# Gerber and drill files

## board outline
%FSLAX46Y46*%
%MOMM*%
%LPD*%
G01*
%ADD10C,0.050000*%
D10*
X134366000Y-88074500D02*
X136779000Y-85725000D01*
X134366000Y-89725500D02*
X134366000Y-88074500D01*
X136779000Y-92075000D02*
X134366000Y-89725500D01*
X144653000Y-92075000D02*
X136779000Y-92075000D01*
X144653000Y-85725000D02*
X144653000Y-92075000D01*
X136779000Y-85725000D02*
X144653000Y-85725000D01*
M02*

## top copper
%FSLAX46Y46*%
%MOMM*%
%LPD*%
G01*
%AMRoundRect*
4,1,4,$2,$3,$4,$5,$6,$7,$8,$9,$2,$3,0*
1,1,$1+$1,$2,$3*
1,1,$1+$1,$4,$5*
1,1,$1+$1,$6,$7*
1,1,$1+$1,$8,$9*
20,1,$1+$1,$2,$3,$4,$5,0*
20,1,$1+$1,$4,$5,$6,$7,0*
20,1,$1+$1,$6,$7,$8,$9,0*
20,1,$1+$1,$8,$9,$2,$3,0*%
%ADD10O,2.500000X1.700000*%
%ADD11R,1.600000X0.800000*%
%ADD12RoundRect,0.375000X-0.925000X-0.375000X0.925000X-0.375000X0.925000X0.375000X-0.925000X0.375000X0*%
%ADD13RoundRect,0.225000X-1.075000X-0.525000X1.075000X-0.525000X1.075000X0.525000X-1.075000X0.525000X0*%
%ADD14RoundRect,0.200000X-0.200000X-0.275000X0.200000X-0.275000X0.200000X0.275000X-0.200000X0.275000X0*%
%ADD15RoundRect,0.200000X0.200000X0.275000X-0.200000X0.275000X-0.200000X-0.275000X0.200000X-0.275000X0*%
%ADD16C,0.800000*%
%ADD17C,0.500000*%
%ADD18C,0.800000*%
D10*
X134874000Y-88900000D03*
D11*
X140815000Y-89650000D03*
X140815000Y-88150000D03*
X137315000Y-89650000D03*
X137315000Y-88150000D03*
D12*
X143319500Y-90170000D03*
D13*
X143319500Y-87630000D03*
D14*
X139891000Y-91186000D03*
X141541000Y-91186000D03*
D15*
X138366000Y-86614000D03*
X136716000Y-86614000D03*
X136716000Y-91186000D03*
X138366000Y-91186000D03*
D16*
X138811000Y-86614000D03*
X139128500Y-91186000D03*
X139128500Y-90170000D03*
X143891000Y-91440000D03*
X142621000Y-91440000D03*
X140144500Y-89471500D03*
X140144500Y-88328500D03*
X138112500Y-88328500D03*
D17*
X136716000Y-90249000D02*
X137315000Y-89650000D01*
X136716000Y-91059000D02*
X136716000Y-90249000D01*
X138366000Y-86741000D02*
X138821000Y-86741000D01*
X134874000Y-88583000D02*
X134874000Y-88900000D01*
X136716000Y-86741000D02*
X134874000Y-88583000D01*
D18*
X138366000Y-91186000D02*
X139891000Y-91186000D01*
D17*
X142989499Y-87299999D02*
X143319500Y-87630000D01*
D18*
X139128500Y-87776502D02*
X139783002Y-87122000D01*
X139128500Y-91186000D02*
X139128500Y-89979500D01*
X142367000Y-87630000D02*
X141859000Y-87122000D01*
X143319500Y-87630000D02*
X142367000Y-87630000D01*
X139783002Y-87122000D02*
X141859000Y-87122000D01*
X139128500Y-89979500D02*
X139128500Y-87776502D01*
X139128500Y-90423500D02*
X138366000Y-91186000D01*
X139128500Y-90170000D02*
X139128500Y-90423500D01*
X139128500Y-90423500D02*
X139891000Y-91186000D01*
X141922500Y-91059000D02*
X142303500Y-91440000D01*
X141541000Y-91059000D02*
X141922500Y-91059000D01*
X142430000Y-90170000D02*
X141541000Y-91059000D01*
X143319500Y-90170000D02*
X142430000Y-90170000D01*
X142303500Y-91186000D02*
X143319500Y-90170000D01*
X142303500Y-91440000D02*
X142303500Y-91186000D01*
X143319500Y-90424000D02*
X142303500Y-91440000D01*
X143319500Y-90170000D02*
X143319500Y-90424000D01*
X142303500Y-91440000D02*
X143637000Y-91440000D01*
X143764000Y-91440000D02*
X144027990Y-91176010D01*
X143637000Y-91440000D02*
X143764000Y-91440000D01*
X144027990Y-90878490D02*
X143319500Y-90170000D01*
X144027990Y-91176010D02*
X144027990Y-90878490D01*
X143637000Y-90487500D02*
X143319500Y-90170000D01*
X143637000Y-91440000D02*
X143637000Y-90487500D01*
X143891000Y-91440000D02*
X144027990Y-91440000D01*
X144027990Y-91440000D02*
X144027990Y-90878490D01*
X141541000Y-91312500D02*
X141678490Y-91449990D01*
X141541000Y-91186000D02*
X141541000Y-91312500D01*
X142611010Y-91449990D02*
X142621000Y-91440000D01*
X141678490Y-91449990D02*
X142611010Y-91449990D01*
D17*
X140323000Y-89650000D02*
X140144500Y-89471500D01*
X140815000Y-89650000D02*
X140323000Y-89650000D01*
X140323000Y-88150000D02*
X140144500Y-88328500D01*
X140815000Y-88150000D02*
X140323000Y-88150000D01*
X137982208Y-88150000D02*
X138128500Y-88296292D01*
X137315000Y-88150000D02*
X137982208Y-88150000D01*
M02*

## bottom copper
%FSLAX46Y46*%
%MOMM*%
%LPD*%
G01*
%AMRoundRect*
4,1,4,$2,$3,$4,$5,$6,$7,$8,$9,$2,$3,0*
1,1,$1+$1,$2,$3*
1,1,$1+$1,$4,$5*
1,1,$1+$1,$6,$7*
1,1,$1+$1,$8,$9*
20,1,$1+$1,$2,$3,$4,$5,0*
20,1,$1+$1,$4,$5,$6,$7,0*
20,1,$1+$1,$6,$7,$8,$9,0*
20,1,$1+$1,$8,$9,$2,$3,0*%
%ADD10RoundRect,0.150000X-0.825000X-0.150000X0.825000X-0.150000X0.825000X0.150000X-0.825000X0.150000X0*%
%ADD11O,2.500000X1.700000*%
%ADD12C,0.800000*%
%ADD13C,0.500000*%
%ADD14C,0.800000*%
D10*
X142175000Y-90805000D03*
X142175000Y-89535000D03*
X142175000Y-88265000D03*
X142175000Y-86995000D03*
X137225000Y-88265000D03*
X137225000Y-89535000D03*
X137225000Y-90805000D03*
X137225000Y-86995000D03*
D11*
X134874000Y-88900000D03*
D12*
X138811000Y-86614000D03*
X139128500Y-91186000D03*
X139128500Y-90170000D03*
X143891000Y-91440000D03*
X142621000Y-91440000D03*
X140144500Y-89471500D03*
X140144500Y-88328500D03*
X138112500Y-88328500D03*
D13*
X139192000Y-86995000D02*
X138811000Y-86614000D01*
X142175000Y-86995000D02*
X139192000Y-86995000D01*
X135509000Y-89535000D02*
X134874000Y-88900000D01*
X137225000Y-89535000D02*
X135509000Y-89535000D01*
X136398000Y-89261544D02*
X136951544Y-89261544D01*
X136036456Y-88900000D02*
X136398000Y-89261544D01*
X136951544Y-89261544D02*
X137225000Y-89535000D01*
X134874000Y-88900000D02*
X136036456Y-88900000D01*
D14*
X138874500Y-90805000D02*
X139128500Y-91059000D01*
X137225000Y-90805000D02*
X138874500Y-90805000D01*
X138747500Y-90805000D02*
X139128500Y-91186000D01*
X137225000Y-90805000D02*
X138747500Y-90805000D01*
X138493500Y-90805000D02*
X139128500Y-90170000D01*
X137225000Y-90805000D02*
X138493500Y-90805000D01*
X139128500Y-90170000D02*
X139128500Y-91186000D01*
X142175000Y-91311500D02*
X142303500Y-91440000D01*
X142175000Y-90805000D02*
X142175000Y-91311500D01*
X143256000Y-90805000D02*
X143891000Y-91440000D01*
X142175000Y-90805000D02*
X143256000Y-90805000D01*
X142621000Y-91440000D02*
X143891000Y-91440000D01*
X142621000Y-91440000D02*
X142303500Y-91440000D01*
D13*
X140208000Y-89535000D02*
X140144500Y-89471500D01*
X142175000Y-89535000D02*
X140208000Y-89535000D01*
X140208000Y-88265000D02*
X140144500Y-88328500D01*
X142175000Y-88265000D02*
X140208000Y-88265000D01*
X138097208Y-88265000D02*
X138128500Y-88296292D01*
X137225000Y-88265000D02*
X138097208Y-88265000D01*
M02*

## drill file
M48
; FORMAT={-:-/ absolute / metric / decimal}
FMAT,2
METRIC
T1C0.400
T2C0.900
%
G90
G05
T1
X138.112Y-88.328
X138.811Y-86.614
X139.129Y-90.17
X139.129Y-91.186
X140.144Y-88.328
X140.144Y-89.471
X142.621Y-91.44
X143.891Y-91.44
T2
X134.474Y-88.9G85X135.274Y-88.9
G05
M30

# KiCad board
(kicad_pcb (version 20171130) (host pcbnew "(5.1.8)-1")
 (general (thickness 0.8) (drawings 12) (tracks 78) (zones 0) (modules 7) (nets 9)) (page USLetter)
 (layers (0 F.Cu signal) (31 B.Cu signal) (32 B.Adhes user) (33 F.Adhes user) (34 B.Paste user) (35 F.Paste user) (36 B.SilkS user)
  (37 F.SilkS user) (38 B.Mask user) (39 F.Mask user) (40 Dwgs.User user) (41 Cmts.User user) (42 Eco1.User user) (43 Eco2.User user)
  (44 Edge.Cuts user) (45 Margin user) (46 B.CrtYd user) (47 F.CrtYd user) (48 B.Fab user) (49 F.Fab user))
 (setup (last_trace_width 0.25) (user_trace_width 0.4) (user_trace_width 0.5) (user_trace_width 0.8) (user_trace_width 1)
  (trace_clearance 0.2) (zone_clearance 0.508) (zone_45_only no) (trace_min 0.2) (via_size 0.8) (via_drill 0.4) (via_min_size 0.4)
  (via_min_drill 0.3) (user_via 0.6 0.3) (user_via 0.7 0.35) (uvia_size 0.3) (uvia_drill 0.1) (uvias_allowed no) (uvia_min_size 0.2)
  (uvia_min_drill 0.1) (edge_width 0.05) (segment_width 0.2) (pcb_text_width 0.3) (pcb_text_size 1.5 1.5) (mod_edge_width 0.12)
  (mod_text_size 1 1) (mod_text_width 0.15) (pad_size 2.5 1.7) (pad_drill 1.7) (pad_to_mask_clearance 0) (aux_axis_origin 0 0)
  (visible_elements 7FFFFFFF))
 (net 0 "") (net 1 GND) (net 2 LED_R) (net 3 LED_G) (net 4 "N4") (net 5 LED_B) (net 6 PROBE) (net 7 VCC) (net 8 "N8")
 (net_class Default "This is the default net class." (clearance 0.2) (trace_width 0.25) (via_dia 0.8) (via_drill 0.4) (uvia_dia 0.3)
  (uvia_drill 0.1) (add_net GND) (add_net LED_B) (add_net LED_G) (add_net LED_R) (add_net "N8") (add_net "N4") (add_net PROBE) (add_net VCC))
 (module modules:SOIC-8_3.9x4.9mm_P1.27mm (layer B.Cu) (at 139.7 88.9)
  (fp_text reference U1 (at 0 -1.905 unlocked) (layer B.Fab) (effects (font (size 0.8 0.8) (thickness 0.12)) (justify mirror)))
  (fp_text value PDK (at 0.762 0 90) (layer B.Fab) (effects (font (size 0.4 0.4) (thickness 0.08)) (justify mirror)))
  (pad 8 smd roundrect (at 2.475 1.905) (size 1.95 0.6) (layers B.Cu B.Paste B.Mask) (roundrect_rratio 0.25) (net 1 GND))
  (pad 7 smd roundrect (at 2.475 0.635) (size 1.95 0.6) (layers B.Cu B.Paste B.Mask) (roundrect_rratio 0.25) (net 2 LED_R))
  (pad 6 smd roundrect (at 2.475 -0.635) (size 1.95 0.6) (layers B.Cu B.Paste B.Mask) (roundrect_rratio 0.25) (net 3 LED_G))
  (pad 5 smd roundrect (at 2.475 -1.905) (size 1.95 0.6) (layers B.Cu B.Paste B.Mask) (roundrect_rratio 0.25) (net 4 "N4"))
  (pad 3 smd roundrect (at -2.475 -0.635) (size 1.95 0.6) (layers B.Cu B.Paste B.Mask) (roundrect_rratio 0.25) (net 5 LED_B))
  (pad 2 smd roundrect (at -2.475 0.635) (size 1.95 0.6) (layers B.Cu B.Paste B.Mask) (roundrect_rratio 0.25) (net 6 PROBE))
  (pad 1 smd roundrect (at -2.475 1.905) (size 1.95 0.6) (layers B.Cu B.Paste B.Mask) (roundrect_rratio 0.25) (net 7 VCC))
  (pad 4 smd roundrect (at -2.475 -1.905) (size 1.95 0.6) (layers B.Cu B.Paste B.Mask) (roundrect_rratio 0.25)))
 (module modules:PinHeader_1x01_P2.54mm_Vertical (layer B.Cu) (at 134.874 88.9)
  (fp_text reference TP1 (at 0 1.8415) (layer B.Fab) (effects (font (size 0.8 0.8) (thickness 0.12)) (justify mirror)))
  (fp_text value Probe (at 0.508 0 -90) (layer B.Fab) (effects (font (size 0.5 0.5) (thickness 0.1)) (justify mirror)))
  (pad 1 thru_hole oval (at 0 0) (size 2.5 1.7) (drill oval 1.7 0.9) (layers *.Cu *.Mask) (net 6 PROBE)))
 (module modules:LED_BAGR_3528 (layer F.Cu) (at 139.065 88.9 180)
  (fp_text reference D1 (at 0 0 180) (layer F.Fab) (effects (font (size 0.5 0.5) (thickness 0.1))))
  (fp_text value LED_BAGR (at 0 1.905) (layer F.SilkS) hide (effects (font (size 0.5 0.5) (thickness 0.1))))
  (pad 4 smd rect (at -1.75 -0.75 180) (size 1.6 0.8) (layers F.Cu F.Paste F.Mask) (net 2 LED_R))
  (pad 3 smd rect (at -1.75 0.75 180) (size 1.6 0.8) (layers F.Cu F.Paste F.Mask) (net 3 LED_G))
  (pad 2 smd rect (at 1.75 -0.75 180) (size 1.6 0.8) (layers F.Cu F.Paste F.Mask) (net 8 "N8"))
  (pad 1 smd rect (at 1.75 0.75 180) (size 1.6 0.8) (layers F.Cu F.Paste F.Mask) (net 5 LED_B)))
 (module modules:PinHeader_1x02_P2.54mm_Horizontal (layer F.Cu) (at 143.3195 87.63)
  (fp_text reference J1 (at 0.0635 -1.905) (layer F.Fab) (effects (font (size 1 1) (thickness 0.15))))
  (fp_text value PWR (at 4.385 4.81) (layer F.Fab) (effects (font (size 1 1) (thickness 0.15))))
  (pad 1 smd roundrect (at 0 2.54) (size 2.6 1.5) (layers F.Cu F.Paste F.Mask) (roundrect_rratio 0.25) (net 1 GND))
  (pad 2 smd roundrect (at 0 0) (size 2.6 1.5) (layers F.Cu F.Paste F.Mask) (roundrect_rratio 0.15) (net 7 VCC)))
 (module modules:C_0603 (layer F.Cu) (at 140.716 91.186)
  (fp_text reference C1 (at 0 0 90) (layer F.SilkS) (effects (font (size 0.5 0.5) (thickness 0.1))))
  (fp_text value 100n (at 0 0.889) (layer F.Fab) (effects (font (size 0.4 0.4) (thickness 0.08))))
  (pad 1 smd roundrect (at -0.825 0) (size 0.8 0.95) (layers F.Cu F.Paste F.Mask) (roundrect_rratio 0.25) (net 7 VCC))
  (pad 2 smd roundrect (at 0.825 0) (size 0.8 0.95) (layers F.Cu F.Paste F.Mask) (roundrect_rratio 0.25) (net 1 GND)))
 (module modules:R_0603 (layer F.Cu) (at 137.541 86.614 180)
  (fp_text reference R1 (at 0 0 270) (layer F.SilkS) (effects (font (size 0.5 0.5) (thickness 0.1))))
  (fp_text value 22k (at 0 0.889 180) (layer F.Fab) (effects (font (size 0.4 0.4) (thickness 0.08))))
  (pad 1 smd roundrect (at -0.825 0 180) (size 0.8 0.95) (layers F.Cu F.Paste F.Mask) (roundrect_rratio 0.25) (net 4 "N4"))
  (pad 2 smd roundrect (at 0.825 0 180) (size 0.8 0.95) (layers F.Cu F.Paste F.Mask) (roundrect_rratio 0.25) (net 6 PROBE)))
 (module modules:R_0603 (layer F.Cu) (at 137.541 91.186 180)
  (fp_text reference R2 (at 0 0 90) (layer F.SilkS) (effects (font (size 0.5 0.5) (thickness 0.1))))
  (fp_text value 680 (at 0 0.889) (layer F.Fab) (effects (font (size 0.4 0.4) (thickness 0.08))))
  (pad 2 smd roundrect (at 0.825 0 180) (size 0.8 0.95) (layers F.Cu F.Paste F.Mask) (roundrect_rratio 0.25) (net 8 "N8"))
  (pad 1 smd roundrect (at -0.825 0 180) (size 0.8 0.95) (layers F.Cu F.Paste F.Mask) (roundrect_rratio 0.25) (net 7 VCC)))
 (gr_line (start 134.366 88.0745) (end 136.779 85.725) (layer Edge.Cuts) (width 0.05))
 (gr_line (start 134.366 89.7255) (end 134.366 88.0745) (layer Edge.Cuts) (width 0.05))
 (gr_line (start 136.779 92.075) (end 134.366 89.7255) (layer Edge.Cuts) (width 0.05))
 (gr_line (start 144.653 92.075) (end 136.779 92.075) (layer Edge.Cuts) (width 0.05))
 (gr_line (start 144.653 85.725) (end 144.653 92.075) (layer Edge.Cuts) (width 0.05))
 (gr_line (start 136.779 85.725) (end 144.653 85.725) (layer Edge.Cuts) (width 0.05))
 (segment (start 136.716 90.249) (end 137.315 89.65) (width 0.5) (layer F.Cu) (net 8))
 (segment (start 136.716 91.059) (end 136.716 90.249) (width 0.5) (layer F.Cu) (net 8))
 (via (at 138.811 86.614) (size 0.8) (drill 0.4) (layers F.Cu B.Cu) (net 4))
 (segment (start 138.366 86.741) (end 138.821 86.741) (width 0.5) (layer F.Cu) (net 4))
 (segment (start 139.192 86.995) (end 138.811 86.614) (width 0.5) (layer B.Cu) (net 4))
 (segment (start 142.175 86.995) (end 139.192 86.995) (width 0.5) (layer B.Cu) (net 4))
 (segment (start 135.509 89.535) (end 134.874 88.9) (width 0.5) (layer B.Cu) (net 6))
 (segment (start 137.225 89.535) (end 135.509 89.535) (width 0.5) (layer B.Cu) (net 6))
 (segment (start 136.398 89.261544) (end 136.951544 89.261544) (width 0.5) (layer B.Cu) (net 6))
 (segment (start 136.036456 88.9) (end 136.398 89.261544) (width 0.5) (layer B.Cu) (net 6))
 (segment (start 136.951544 89.261544) (end 137.225 89.535) (width 0.5) (layer B.Cu) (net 6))
 (segment (start 134.874 88.9) (end 136.036456 88.9) (width 0.5) (layer B.Cu) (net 6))
 (segment (start 134.874 88.583) (end 134.874 88.9) (width 0.5) (layer F.Cu) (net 6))
 (segment (start 136.716 86.741) (end 134.874 88.583) (width 0.5) (layer F.Cu) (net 6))
 (via (at 139.1285 91.186) (size 0.8) (drill 0.4) (layers F.Cu B.Cu) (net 7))
 (segment (start 138.8745 90.805) (end 139.1285 91.059) (width 0.8) (layer B.Cu) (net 7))
 (segment (start 137.225 90.805) (end 138.8745 90.805) (width 0.8) (layer B.Cu) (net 7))
 (segment (start 138.366 91.186) (end 139.891 91.186) (width 0.8) (layer F.Cu) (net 7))
 (segment (start 142.989499 87.299999) (end 143.3195 87.63) (width 0.5) (layer F.Cu) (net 7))
 (segment (start 139.1285 87.776502) (end 139.783002 87.122) (width 0.8) (layer F.Cu) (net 7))
 (segment (start 139.1285 91.186) (end 139.1285 89.9795) (width 0.8) (layer F.Cu) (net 7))
 (segment (start 142.367 87.63) (end 141.859 87.122) (width 0.8) (layer F.Cu) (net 7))
 (segment (start 143.3195 87.63) (end 142.367 87.63) (width 0.8) (layer F.Cu) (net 7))
 (segment (start 139.783002 87.122) (end 141.859 87.122) (width 0.8) (layer F.Cu) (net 7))
 (segment (start 139.1285 89.9795) (end 139.1285 87.776502) (width 0.8) (layer F.Cu) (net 7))
 (via (at 139.1285 90.17) (size 0.8) (drill 0.4) (layers F.Cu B.Cu) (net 7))
 (segment (start 138.7475 90.805) (end 139.1285 91.186) (width 0.8) (layer B.Cu) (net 7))
 (segment (start 137.225 90.805) (end 138.7475 90.805) (width 0.8) (layer B.Cu) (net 7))
 (segment (start 138.4935 90.805) (end 139.1285 90.17) (width 0.8) (layer B.Cu) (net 7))
 (segment (start 137.225 90.805) (end 138.4935 90.805) (width 0.8) (layer B.Cu) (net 7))
 (segment (start 139.1285 90.17) (end 139.1285 91.186) (width 0.8) (layer B.Cu) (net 7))
 (segment (start 139.1285 90.4235) (end 138.366 91.186) (width 0.8) (layer F.Cu) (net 7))
 (segment (start 139.1285 90.17) (end 139.1285 90.4235) (width 0.8) (layer F.Cu) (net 7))
 (segment (start 139.1285 90.4235) (end 139.891 91.186) (width 0.8) (layer F.Cu) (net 7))
 (via (at 143.891 91.44) (size 0.8) (drill 0.4) (layers F.Cu B.Cu) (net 1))
 (via (at 142.621 91.44) (size 0.8) (drill 0.4) (layers F.Cu B.Cu) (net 1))
 (segment (start 142.175 91.3115) (end 142.3035 91.44) (width 0.8) (layer B.Cu) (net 1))
 (segment (start 142.175 90.805) (end 142.175 91.3115) (width 0.8) (layer B.Cu) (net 1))
 (segment (start 141.9225 91.059) (end 142.3035 91.44) (width 0.8) (layer F.Cu) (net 1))
 (segment (start 141.541 91.059) (end 141.9225 91.059) (width 0.8) (layer F.Cu) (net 1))
 (segment (start 142.43 90.17) (end 141.541 91.059) (width 0.8) (layer F.Cu) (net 1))
 (segment (start 143.3195 90.17) (end 142.43 90.17) (width 0.8) (layer F.Cu) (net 1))
 (segment (start 142.3035 91.186) (end 143.3195 90.17) (width 0.8) (layer F.Cu) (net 1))
 (segment (start 142.3035 91.44) (end 142.3035 91.186) (width 0.8) (layer F.Cu) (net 1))
 (segment (start 143.3195 90.424) (end 142.3035 91.44) (width 0.8) (layer F.Cu) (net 1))
 (segment (start 143.3195 90.17) (end 143.3195 90.424) (width 0.8) (layer F.Cu) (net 1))
 (segment (start 142.3035 91.44) (end 143.637 91.44) (width 0.8) (layer F.Cu) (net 1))
 (segment (start 143.764 91.44) (end 144.02799 91.17601) (width 0.8) (layer F.Cu) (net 1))
 (segment (start 143.637 91.44) (end 143.764 91.44) (width 0.8) (layer F.Cu) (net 1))
 (segment (start 144.02799 90.87849) (end 143.3195 90.17) (width 0.8) (layer F.Cu) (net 1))
 (segment (start 144.02799 91.17601) (end 144.02799 90.87849) (width 0.8) (layer F.Cu) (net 1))
 (segment (start 143.637 90.4875) (end 143.3195 90.17) (width 0.8) (layer F.Cu) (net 1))
 (segment (start 143.637 91.44) (end 143.637 90.4875) (width 0.8) (layer F.Cu) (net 1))
 (segment (start 143.891 91.44) (end 144.02799 91.44) (width 0.8) (layer F.Cu) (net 1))
 (segment (start 144.02799 91.44) (end 144.02799 90.87849) (width 0.8) (layer F.Cu) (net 1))
 (segment (start 143.256 90.805) (end 143.891 91.44) (width 0.8) (layer B.Cu) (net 1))
 (segment (start 142.175 90.805) (end 143.256 90.805) (width 0.8) (layer B.Cu) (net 1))
 (segment (start 142.621 91.44) (end 143.891 91.44) (width 0.8) (layer B.Cu) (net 1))
 (segment (start 141.541 91.3125) (end 141.67849 91.44999) (width 0.8) (layer F.Cu) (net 1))
 (segment (start 141.541 91.186) (end 141.541 91.3125) (width 0.8) (layer F.Cu) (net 1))
 (segment (start 142.61101 91.44999) (end 142.621 91.44) (width 0.8) (layer F.Cu) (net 1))
 (segment (start 141.67849 91.44999) (end 142.61101 91.44999) (width 0.8) (layer F.Cu) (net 1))
 (segment (start 142.621 91.44) (end 142.3035 91.44) (width 0.8) (layer B.Cu) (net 1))
 (via (at 140.1445 89.4715) (size 0.8) (drill 0.4) (layers F.Cu B.Cu) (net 2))
 (segment (start 140.323 89.65) (end 140.1445 89.4715) (width 0.5) (layer F.Cu) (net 2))
 (segment (start 140.815 89.65) (end 140.323 89.65) (width 0.5) (layer F.Cu) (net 2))
 (segment (start 140.208 89.535) (end 140.1445 89.4715) (width 0.5) (layer B.Cu) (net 2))
 (segment (start 142.175 89.535) (end 140.208 89.535) (width 0.5) (layer B.Cu) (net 2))
 (via (at 140.1445 88.3285) (size 0.8) (drill 0.4) (layers F.Cu B.Cu) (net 3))
 (segment (start 140.323 88.15) (end 140.1445 88.3285) (width 0.5) (layer F.Cu) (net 3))
 (segment (start 140.815 88.15) (end 140.323 88.15) (width 0.5) (layer F.Cu) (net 3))
 (segment (start 140.208 88.265) (end 140.1445 88.3285) (width 0.5) (layer B.Cu) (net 3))
 (segment (start 142.175 88.265) (end 140.208 88.265) (width 0.5) (layer B.Cu) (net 3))
 (via (at 138.1125 88.3285) (size 0.8) (drill 0.4) (layers F.Cu B.Cu) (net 5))
 (segment (start 137.982208 88.15) (end 138.1285 88.296292) (width 0.5) (layer F.Cu) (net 5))
 (segment (start 137.315 88.15) (end 137.982208 88.15) (width 0.5) (layer F.Cu) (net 5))
 (segment (start 138.097208 88.265) (end 138.1285 88.296292) (width 0.5) (layer B.Cu) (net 5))
 (segment (start 137.225 88.265) (end 138.097208 88.265) (width 0.5) (layer B.Cu) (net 5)))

